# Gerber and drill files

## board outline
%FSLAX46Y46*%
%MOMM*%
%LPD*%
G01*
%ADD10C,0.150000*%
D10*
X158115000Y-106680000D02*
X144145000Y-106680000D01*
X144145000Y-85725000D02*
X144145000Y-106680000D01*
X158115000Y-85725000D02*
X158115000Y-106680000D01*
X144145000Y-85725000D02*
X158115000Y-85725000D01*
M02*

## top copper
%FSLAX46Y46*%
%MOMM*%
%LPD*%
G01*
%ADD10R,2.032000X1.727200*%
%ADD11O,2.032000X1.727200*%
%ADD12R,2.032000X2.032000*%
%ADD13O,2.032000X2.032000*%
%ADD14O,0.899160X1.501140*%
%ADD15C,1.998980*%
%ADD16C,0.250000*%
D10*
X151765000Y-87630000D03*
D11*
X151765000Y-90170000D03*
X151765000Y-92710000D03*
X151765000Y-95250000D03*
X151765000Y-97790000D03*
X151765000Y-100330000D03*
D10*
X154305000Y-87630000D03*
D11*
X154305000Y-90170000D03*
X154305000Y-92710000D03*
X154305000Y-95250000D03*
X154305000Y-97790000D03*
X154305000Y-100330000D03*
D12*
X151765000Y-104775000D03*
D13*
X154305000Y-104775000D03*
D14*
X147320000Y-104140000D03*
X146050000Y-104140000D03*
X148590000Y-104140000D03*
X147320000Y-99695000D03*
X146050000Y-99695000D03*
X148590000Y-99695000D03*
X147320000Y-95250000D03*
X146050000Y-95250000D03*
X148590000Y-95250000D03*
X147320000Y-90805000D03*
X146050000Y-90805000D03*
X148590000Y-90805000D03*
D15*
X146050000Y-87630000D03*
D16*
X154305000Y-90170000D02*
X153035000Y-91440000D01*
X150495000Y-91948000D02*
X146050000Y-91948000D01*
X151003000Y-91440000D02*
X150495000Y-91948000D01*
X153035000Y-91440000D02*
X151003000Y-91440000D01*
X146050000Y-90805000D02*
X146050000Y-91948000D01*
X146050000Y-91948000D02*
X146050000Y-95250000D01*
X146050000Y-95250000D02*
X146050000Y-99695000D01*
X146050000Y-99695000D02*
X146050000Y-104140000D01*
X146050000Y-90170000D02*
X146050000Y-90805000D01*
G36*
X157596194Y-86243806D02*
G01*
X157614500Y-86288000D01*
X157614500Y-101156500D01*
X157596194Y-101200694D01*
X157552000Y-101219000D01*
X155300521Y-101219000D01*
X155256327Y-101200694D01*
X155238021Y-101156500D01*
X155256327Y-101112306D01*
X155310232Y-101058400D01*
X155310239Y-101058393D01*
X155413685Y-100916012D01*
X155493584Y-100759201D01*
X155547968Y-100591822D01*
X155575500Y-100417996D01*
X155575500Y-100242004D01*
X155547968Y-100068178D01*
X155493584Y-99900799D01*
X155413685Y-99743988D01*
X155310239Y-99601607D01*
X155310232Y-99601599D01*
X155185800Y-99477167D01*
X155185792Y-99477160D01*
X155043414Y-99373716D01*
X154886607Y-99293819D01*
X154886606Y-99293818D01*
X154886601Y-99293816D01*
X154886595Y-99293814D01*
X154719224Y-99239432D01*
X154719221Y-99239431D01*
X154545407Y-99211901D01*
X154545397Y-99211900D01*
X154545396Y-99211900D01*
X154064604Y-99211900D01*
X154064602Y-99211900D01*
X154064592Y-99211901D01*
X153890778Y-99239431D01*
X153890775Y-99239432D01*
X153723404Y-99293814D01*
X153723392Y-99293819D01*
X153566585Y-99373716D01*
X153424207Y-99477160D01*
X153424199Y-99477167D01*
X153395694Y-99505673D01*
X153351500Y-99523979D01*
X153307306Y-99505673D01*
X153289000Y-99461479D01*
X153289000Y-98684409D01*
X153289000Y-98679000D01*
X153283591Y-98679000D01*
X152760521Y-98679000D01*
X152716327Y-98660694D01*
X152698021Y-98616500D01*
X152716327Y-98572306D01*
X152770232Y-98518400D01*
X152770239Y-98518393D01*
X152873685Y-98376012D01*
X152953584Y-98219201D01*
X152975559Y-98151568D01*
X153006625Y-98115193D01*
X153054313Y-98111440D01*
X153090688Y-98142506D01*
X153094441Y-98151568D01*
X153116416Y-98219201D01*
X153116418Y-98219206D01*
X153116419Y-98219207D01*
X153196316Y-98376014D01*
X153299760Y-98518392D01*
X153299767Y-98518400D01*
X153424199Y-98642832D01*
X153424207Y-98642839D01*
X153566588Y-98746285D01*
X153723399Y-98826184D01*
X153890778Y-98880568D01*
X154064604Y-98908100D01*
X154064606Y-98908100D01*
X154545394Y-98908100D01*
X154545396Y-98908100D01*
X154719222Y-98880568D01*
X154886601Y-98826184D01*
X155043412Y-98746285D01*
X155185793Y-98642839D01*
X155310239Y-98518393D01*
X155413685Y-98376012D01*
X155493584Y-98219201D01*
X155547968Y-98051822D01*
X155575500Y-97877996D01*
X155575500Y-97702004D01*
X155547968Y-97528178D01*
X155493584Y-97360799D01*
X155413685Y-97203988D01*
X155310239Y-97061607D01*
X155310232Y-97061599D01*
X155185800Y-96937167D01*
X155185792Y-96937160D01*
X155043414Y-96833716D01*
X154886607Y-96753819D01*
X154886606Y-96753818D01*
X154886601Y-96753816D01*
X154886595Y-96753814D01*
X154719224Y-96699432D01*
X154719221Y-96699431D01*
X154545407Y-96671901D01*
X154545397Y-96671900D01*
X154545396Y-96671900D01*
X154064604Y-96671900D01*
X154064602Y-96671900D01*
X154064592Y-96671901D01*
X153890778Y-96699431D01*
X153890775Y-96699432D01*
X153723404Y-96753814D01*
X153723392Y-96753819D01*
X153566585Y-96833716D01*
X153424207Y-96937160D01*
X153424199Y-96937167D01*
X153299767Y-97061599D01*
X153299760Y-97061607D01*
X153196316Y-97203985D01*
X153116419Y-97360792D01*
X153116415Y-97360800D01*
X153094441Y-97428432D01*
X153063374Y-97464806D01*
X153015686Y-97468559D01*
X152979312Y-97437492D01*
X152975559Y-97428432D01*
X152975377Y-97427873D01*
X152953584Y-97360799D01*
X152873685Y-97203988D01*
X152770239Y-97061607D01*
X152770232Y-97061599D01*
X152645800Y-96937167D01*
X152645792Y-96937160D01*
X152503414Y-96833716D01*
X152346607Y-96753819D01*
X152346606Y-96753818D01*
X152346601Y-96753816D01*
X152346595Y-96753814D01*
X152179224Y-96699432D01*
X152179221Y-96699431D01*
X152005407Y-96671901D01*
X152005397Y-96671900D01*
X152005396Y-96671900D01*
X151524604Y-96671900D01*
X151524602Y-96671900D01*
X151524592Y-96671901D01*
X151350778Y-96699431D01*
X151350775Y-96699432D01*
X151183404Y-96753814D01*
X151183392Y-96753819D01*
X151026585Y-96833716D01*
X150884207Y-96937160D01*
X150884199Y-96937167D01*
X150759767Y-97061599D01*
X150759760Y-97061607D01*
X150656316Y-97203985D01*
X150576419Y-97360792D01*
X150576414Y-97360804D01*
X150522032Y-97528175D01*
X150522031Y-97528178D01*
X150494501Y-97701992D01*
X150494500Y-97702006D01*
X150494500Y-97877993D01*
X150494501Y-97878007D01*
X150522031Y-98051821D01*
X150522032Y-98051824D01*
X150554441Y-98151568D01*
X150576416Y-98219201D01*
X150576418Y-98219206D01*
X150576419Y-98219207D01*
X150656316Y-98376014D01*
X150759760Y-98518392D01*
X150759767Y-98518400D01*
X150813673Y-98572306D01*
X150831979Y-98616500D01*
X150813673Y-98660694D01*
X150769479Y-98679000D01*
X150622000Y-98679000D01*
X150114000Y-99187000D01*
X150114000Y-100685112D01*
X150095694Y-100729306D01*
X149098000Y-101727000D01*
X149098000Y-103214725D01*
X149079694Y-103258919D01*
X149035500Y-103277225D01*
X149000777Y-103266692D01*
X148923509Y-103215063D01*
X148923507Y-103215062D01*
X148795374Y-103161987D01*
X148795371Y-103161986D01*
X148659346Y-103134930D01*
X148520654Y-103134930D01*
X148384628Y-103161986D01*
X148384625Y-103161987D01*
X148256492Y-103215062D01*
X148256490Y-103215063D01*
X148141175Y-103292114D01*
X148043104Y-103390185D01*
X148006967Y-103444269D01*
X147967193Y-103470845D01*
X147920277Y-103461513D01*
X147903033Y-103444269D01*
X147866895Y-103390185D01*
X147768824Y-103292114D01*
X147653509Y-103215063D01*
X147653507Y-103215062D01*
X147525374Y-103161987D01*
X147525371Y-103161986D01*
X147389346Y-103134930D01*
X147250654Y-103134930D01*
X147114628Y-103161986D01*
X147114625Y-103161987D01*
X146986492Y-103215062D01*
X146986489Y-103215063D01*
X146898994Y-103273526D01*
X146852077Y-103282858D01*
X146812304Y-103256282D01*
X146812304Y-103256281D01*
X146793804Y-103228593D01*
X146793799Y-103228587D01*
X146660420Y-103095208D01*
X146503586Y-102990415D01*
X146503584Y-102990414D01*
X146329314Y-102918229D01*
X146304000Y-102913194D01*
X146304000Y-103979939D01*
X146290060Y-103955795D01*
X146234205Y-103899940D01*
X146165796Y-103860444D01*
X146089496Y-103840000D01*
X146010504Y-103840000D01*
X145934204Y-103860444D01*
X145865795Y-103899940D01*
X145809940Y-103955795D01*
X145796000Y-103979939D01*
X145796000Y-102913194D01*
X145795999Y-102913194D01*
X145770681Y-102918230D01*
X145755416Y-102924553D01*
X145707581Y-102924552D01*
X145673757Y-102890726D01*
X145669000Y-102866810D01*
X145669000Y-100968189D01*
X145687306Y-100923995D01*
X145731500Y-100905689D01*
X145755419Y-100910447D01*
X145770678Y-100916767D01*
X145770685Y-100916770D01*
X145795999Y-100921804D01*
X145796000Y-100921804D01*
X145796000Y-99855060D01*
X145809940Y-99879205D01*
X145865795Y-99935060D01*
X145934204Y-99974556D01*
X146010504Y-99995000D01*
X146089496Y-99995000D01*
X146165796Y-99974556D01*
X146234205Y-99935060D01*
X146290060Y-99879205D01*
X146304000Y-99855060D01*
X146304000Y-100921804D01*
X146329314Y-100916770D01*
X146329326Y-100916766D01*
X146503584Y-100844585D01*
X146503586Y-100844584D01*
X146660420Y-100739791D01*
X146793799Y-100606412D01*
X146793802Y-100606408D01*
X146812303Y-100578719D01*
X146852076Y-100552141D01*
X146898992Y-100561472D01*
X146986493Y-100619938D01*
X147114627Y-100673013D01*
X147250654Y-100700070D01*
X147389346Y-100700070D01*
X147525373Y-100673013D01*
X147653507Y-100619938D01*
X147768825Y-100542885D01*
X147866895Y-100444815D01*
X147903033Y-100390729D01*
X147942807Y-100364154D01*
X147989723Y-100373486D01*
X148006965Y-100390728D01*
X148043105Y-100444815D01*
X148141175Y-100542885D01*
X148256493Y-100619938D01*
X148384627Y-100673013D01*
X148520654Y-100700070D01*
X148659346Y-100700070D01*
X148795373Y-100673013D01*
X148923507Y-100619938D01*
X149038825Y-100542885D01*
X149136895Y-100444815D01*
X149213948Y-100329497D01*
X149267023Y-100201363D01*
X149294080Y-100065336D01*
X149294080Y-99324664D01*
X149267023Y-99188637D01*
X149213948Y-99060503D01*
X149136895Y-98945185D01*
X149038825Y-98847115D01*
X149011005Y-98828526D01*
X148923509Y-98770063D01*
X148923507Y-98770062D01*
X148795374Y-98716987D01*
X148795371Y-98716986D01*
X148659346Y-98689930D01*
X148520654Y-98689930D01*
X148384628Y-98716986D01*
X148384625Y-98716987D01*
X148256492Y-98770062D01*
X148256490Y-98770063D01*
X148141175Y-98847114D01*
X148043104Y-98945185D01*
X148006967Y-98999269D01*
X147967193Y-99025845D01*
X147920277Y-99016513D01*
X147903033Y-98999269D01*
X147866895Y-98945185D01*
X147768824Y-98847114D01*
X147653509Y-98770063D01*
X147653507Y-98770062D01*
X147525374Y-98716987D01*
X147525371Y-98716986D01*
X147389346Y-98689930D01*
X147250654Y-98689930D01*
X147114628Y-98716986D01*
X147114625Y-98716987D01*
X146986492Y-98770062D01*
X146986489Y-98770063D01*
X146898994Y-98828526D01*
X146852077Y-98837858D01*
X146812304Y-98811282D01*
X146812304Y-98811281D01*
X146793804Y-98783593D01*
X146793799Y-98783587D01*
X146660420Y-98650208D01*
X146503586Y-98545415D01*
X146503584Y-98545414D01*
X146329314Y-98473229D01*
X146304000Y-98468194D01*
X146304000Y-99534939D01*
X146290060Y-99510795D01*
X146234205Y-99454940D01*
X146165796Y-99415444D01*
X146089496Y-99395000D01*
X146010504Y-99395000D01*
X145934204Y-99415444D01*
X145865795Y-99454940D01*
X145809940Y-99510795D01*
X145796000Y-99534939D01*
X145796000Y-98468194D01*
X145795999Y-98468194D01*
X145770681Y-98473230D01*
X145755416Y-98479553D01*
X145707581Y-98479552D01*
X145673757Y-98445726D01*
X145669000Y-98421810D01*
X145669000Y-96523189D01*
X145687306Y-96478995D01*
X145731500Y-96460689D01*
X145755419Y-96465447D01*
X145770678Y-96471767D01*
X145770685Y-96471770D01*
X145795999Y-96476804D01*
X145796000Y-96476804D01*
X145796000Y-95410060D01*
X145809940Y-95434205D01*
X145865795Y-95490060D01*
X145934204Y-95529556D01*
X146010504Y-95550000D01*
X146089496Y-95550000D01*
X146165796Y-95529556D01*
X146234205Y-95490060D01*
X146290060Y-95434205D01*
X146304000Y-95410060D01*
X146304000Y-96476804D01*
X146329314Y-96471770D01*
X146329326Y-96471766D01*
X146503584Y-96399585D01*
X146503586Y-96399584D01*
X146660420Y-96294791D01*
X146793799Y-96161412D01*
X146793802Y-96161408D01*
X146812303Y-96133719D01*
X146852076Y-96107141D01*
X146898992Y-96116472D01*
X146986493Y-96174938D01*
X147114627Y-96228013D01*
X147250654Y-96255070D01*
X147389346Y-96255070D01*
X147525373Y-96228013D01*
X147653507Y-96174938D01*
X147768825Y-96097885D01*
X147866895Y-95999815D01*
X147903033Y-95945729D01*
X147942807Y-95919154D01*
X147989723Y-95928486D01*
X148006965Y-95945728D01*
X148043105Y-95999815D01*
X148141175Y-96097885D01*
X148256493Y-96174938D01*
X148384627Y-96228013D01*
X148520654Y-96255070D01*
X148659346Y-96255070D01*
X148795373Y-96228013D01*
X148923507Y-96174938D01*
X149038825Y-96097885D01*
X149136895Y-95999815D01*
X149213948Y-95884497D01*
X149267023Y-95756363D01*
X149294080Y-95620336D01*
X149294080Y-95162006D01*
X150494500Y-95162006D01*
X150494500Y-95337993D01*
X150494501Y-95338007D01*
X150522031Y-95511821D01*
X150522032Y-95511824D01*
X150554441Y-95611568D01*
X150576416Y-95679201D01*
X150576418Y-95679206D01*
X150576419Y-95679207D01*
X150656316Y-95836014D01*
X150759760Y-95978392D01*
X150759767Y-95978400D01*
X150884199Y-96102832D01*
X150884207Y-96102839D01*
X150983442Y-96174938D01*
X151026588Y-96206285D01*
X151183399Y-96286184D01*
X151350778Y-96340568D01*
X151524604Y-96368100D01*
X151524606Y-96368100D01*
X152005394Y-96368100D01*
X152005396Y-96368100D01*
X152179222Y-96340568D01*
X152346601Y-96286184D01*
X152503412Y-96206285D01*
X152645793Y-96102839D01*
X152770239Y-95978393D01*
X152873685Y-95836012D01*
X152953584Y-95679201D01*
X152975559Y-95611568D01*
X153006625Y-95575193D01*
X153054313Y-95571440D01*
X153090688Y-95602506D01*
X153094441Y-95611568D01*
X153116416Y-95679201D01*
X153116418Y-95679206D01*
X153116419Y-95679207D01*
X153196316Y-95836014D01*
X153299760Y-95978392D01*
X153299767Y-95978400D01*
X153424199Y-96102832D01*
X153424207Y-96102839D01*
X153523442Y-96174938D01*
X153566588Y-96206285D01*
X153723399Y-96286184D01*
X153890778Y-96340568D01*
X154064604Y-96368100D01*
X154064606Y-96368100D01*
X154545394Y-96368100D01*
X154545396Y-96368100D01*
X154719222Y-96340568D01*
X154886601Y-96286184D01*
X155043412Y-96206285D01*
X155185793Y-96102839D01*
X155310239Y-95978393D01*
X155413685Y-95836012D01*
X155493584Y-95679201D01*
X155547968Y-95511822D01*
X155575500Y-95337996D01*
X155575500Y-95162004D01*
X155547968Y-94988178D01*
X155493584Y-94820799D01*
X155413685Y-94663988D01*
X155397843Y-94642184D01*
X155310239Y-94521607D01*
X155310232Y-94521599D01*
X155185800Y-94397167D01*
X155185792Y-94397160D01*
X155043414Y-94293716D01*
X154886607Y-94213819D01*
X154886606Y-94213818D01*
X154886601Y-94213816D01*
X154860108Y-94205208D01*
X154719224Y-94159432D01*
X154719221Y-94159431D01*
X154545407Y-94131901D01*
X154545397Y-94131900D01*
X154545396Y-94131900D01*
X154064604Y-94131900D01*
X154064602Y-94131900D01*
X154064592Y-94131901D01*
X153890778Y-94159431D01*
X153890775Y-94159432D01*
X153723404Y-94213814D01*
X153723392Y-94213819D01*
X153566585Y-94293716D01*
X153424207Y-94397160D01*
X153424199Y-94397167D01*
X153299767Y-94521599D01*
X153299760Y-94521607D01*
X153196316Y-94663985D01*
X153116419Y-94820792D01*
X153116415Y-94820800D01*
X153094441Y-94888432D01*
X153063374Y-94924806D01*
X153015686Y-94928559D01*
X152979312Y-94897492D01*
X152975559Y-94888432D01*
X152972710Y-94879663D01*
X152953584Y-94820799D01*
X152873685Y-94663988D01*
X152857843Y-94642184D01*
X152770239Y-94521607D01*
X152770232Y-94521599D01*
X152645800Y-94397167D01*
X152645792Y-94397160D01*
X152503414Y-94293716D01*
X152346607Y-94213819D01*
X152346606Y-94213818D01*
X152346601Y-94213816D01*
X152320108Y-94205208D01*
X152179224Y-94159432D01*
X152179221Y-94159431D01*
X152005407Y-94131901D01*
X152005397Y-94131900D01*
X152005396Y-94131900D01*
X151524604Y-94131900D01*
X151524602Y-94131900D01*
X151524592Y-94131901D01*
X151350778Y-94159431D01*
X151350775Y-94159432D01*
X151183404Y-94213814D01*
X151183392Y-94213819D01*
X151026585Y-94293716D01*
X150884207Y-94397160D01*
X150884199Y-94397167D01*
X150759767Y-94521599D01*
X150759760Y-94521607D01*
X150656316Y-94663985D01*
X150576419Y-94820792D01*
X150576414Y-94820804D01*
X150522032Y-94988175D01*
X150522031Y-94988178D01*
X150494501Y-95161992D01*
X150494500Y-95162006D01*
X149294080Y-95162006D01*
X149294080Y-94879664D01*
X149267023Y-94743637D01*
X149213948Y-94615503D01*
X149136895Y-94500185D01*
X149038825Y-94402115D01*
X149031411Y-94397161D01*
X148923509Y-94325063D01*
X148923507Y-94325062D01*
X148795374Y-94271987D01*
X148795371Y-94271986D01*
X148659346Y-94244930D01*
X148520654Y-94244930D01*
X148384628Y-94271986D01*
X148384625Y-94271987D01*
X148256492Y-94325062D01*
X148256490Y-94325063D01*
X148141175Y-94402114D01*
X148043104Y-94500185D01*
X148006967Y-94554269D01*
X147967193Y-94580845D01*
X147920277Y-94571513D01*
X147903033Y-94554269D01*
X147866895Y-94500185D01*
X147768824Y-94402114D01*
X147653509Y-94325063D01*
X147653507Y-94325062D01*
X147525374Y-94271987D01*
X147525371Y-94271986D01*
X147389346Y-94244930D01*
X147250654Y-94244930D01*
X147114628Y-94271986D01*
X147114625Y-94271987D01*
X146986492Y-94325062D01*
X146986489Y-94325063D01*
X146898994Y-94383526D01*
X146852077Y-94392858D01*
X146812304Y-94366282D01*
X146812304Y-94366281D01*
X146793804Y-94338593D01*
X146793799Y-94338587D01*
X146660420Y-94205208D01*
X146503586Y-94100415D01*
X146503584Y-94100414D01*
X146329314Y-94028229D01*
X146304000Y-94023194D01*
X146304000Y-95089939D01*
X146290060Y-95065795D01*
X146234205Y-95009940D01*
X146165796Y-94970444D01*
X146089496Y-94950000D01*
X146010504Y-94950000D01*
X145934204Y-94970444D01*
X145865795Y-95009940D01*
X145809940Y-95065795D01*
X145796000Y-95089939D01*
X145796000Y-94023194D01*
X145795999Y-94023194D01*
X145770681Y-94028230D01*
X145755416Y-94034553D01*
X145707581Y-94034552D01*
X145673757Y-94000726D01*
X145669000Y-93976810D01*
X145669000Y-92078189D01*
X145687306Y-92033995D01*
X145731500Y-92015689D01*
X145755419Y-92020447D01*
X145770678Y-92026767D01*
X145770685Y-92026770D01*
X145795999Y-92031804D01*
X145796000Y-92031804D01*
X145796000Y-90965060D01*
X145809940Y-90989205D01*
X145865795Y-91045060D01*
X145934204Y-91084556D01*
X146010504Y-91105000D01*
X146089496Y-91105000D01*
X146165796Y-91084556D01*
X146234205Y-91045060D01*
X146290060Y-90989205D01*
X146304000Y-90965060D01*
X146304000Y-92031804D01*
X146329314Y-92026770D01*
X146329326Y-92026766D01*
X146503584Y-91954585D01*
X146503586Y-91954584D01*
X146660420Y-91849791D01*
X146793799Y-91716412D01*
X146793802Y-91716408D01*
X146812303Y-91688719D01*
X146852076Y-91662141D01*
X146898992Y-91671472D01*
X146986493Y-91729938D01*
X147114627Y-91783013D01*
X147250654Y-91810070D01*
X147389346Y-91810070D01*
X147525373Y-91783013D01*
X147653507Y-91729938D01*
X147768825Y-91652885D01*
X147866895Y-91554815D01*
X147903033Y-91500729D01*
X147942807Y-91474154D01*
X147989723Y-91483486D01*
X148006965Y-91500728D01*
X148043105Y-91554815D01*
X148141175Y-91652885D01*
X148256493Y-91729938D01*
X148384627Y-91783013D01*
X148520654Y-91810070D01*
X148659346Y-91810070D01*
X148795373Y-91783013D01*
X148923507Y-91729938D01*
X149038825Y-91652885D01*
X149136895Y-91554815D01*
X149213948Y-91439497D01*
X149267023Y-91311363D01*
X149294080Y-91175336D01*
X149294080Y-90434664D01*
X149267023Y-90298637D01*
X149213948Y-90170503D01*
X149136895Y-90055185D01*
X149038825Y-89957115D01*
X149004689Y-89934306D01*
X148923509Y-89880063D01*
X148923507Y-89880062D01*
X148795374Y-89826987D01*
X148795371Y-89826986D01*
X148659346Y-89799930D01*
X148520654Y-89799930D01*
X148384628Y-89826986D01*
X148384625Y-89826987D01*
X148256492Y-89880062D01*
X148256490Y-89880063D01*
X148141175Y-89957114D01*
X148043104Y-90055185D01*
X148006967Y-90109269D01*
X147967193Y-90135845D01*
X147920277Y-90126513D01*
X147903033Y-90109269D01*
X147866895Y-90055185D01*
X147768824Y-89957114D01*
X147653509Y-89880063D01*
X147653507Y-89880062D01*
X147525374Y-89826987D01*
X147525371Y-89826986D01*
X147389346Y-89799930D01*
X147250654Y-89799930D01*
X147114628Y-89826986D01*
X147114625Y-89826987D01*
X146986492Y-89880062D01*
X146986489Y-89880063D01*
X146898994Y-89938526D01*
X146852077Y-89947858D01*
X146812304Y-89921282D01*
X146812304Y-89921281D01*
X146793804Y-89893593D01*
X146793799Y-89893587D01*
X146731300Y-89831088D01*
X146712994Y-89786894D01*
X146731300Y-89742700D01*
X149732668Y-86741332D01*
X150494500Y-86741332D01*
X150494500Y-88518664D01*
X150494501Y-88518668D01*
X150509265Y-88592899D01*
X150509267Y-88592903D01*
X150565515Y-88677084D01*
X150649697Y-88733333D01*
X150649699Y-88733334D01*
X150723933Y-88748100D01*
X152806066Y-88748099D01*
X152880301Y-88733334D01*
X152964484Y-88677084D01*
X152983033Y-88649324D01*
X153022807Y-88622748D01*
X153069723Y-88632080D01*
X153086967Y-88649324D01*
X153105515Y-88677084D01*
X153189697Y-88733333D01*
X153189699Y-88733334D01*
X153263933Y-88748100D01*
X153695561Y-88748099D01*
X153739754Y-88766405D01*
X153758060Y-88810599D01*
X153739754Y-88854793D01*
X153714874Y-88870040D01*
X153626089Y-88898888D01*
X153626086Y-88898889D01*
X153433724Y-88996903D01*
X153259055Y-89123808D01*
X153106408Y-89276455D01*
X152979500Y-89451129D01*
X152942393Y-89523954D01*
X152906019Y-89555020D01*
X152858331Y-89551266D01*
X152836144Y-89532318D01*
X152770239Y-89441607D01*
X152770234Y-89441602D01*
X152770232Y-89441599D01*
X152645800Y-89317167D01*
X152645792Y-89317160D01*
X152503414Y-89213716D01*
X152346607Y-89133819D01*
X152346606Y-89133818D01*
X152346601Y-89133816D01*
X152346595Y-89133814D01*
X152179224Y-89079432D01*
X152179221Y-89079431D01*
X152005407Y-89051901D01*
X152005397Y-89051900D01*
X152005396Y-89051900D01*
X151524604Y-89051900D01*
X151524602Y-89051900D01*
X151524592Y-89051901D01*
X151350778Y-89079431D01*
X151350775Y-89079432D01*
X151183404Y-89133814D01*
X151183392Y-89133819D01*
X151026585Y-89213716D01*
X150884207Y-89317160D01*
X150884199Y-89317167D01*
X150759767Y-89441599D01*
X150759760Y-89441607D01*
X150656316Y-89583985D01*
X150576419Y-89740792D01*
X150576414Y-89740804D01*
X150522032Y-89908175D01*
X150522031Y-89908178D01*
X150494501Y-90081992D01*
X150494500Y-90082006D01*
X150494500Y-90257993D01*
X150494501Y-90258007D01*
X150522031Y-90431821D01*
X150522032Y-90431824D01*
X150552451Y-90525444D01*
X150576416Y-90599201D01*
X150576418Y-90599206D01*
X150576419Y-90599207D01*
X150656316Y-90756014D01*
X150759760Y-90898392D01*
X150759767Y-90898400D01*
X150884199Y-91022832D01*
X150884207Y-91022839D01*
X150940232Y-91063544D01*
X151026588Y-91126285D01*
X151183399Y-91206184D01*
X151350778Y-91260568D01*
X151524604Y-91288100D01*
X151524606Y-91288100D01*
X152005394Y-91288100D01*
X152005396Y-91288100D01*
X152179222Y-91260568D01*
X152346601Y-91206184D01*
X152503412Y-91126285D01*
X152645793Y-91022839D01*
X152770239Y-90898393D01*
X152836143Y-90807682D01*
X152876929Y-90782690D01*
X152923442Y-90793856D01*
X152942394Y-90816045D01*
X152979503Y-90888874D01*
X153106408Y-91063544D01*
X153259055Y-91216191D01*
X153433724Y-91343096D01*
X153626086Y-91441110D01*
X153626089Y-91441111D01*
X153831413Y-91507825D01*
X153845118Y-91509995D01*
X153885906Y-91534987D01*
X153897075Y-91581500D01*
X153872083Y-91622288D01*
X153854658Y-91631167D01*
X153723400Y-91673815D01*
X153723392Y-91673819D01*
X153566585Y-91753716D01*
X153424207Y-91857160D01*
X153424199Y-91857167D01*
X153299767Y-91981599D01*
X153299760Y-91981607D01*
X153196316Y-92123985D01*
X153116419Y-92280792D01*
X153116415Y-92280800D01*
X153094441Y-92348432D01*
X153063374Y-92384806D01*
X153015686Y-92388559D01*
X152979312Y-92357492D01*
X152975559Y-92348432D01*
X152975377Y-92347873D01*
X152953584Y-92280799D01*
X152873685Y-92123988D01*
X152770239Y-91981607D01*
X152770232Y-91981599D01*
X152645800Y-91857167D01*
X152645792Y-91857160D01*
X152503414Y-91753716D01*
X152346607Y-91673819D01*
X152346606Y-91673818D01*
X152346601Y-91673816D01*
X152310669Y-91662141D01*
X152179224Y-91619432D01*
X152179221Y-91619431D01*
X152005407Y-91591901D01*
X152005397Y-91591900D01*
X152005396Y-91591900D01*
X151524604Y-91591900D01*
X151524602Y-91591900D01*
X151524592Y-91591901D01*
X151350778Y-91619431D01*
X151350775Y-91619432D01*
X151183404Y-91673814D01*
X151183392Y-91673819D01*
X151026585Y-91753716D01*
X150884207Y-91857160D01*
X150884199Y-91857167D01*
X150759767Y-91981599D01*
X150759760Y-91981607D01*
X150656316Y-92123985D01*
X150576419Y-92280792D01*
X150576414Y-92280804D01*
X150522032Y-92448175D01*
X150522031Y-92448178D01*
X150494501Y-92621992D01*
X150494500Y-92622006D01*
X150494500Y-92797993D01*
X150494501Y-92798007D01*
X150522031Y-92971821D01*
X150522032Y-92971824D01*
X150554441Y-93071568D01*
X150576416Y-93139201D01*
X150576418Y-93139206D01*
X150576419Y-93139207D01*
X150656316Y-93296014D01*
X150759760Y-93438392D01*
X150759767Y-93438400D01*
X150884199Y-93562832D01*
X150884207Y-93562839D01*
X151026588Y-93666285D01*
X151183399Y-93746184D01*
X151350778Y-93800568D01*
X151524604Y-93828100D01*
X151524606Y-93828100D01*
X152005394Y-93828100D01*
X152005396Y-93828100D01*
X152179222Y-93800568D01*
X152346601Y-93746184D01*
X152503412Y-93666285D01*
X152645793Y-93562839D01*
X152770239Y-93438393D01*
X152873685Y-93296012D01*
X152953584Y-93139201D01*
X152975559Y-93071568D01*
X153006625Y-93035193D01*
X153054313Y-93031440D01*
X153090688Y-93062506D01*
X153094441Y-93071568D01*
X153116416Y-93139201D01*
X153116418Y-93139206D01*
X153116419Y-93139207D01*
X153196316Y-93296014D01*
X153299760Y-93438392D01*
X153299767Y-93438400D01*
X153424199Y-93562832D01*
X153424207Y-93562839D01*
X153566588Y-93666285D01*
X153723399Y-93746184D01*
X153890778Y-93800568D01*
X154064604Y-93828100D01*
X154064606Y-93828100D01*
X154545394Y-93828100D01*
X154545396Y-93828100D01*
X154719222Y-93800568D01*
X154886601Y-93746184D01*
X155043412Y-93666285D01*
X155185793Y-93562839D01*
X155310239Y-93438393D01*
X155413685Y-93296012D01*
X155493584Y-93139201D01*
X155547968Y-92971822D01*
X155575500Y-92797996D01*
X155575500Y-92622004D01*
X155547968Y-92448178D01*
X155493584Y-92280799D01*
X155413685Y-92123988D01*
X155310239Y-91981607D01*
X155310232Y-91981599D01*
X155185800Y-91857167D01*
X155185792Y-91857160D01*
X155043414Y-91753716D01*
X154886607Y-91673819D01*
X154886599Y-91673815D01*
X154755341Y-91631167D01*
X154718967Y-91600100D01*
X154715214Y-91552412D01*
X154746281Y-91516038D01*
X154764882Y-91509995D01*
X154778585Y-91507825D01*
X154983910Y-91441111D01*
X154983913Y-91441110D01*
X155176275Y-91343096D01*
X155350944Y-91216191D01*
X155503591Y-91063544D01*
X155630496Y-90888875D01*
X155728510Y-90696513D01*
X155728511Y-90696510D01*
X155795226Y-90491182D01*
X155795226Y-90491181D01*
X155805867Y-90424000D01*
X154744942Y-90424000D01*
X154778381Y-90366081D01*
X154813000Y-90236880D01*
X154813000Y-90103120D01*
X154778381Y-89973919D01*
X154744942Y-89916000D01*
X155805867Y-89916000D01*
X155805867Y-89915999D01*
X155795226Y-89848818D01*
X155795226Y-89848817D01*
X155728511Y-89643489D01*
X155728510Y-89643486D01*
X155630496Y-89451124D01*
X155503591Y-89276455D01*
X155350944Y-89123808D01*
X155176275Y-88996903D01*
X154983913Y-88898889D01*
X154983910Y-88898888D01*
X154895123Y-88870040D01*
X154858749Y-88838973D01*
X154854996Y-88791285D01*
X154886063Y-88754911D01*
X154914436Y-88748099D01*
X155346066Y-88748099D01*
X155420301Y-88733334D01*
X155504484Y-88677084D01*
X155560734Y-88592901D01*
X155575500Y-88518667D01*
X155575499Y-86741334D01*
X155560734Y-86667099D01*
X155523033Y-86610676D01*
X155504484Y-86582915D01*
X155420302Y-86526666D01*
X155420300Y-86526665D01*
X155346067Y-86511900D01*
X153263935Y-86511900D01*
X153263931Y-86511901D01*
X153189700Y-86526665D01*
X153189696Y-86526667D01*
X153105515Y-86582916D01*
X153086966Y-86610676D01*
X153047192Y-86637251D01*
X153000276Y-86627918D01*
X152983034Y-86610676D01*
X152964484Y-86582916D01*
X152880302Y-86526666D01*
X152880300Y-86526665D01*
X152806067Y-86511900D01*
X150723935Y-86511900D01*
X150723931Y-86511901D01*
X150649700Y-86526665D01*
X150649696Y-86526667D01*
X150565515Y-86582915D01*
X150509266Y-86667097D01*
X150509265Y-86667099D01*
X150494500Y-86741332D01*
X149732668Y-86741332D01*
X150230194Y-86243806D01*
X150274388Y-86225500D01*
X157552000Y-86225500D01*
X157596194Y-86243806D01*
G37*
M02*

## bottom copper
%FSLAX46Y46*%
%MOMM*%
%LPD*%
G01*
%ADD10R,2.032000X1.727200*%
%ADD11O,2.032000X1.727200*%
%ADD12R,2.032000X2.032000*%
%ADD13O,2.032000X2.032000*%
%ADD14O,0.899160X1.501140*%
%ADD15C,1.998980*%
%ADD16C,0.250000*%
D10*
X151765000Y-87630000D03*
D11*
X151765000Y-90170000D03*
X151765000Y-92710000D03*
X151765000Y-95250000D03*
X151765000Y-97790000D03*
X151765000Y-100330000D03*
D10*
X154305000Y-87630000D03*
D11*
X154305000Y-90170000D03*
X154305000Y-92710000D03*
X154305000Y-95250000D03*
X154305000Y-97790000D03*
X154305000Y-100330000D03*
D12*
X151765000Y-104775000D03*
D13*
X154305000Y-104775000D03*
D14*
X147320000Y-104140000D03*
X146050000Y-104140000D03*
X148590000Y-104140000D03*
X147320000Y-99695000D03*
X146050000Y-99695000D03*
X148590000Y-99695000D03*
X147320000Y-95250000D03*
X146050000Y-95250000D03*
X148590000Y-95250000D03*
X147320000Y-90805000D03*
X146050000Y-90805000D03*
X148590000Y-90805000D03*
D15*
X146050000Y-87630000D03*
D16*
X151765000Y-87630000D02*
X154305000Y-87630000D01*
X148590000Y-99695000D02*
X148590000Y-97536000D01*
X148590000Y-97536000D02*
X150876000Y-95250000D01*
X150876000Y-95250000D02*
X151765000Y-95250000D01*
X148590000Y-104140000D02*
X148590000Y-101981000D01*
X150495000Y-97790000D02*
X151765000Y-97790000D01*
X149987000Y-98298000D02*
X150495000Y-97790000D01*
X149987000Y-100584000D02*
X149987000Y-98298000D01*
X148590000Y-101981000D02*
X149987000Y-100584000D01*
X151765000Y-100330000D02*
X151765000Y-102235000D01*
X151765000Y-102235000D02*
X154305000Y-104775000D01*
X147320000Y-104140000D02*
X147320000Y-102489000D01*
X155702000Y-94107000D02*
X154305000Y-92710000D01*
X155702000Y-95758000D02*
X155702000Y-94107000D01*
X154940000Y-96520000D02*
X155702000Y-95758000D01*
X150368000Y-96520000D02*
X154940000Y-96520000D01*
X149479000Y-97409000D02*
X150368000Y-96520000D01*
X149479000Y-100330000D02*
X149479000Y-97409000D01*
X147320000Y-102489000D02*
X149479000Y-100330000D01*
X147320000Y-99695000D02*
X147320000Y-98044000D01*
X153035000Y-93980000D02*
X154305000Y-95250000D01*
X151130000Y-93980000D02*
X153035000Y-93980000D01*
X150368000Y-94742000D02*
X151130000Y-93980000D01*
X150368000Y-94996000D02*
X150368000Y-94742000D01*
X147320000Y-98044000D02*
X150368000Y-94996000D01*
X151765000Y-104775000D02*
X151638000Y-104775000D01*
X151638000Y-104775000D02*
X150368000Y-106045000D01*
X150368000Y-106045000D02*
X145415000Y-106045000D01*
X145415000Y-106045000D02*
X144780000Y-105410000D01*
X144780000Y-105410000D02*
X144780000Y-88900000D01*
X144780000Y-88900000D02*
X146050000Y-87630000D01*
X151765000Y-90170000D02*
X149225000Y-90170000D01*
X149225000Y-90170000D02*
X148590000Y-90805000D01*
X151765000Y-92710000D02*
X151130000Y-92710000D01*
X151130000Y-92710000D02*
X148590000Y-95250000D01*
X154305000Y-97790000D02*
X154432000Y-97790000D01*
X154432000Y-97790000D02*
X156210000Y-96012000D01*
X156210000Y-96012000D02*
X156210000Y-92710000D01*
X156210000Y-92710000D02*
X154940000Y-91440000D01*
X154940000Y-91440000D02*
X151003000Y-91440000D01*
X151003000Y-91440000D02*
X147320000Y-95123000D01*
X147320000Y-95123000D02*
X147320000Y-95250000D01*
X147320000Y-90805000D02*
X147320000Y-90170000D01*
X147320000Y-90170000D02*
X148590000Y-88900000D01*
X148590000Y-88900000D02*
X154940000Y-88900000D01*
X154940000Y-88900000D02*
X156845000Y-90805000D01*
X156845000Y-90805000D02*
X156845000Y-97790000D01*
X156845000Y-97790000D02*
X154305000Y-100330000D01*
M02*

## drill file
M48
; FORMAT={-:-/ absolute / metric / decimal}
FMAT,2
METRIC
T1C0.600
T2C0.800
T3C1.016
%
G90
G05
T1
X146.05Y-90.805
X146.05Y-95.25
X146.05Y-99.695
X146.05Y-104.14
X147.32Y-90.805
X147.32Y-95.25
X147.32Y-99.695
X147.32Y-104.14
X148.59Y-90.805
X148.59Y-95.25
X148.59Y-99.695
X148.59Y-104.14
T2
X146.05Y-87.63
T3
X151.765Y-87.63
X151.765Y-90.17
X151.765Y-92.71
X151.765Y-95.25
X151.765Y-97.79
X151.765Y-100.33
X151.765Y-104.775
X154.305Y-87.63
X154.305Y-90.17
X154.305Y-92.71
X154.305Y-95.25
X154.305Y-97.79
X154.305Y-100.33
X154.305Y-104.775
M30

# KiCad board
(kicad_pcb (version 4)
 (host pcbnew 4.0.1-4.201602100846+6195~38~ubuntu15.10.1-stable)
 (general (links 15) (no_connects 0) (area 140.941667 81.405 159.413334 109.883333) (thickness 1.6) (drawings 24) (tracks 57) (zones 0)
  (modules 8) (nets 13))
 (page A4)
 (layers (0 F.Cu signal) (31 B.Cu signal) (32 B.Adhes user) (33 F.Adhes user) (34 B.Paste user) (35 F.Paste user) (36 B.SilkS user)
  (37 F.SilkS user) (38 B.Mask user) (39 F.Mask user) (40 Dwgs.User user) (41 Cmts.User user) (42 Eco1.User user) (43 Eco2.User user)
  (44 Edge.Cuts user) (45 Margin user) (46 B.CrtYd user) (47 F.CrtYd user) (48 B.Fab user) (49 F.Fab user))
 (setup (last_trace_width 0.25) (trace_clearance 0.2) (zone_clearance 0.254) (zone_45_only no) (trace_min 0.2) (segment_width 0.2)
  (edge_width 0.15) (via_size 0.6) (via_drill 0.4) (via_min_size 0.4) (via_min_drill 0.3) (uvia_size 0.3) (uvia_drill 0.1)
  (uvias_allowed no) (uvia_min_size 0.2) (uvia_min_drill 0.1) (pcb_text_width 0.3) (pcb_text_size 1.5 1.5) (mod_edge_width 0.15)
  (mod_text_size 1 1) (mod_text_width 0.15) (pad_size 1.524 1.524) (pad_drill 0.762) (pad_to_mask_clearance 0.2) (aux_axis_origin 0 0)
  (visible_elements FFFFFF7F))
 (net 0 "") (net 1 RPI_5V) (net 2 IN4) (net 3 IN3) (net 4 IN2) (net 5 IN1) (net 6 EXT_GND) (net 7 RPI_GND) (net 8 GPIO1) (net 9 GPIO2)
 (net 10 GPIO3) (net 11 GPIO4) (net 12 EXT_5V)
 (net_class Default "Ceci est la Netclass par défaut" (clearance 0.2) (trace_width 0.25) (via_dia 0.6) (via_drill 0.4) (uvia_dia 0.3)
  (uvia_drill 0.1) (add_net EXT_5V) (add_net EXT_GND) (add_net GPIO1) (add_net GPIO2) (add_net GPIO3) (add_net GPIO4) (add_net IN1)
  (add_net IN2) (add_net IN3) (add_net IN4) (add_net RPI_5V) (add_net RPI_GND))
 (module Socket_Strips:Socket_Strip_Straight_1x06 (layer B.Cu) (at 151.765 87.63 270)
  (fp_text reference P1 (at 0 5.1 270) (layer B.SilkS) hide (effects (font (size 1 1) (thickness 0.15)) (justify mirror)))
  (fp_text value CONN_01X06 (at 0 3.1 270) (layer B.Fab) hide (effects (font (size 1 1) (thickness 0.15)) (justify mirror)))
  (pad 1 thru_hole rect (at 0 0 270) (size 1.7272 2.032) (drill 1.016) (layers *.Cu *.Mask B.SilkS) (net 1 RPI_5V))
  (pad 2 thru_hole oval (at 2.54 0 270) (size 1.7272 2.032) (drill 1.016) (layers *.Cu *.Mask B.SilkS) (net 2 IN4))
  (pad 3 thru_hole oval (at 5.08 0 270) (size 1.7272 2.032) (drill 1.016) (layers *.Cu *.Mask B.SilkS) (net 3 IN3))
  (pad 4 thru_hole oval (at 7.62 0 270) (size 1.7272 2.032) (drill 1.016) (layers *.Cu *.Mask B.SilkS) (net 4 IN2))
  (pad 5 thru_hole oval (at 10.16 0 270) (size 1.7272 2.032) (drill 1.016) (layers *.Cu *.Mask B.SilkS) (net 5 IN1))
  (pad 6 thru_hole oval (at 12.7 0 270) (size 1.7272 2.032) (drill 1.016) (layers *.Cu *.Mask B.SilkS) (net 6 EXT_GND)))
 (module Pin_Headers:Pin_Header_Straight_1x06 (layer F.Cu) (at 154.305 87.63)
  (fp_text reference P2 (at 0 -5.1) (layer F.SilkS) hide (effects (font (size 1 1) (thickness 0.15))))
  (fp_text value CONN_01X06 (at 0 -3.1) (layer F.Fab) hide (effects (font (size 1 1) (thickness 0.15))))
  (pad 1 thru_hole rect (at 0 0) (size 2.032 1.7272) (drill 1.016) (layers *.Cu *.Mask F.SilkS) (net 1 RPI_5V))
  (pad 2 thru_hole oval (at 0 2.54) (size 2.032 1.7272) (drill 1.016) (layers *.Cu *.Mask F.SilkS) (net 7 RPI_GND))
  (pad 3 thru_hole oval (at 0 5.08) (size 2.032 1.7272) (drill 1.016) (layers *.Cu *.Mask F.SilkS) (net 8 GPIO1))
  (pad 4 thru_hole oval (at 0 7.62) (size 2.032 1.7272) (drill 1.016) (layers *.Cu *.Mask F.SilkS) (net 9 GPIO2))
  (pad 5 thru_hole oval (at 0 10.16) (size 2.032 1.7272) (drill 1.016) (layers *.Cu *.Mask F.SilkS) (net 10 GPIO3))
  (pad 6 thru_hole oval (at 0 12.7) (size 2.032 1.7272) (drill 1.016) (layers *.Cu *.Mask F.SilkS) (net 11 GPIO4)))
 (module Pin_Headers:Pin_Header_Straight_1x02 (layer F.Cu) (at 151.765 104.775 90)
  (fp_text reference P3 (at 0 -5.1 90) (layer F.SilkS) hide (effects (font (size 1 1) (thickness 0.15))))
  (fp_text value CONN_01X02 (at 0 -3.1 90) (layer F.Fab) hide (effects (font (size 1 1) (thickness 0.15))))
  (pad 1 thru_hole rect (at 0 0 90) (size 2.032 2.032) (drill 1.016) (layers *.Cu *.Mask F.SilkS) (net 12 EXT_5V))
  (pad 2 thru_hole oval (at 0 2.54 90) (size 2.032 2.032) (drill 1.016) (layers *.Cu *.Mask F.SilkS) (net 6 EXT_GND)))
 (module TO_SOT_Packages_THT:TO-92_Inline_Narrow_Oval (layer F.Cu) (at 148.59 104.14 180)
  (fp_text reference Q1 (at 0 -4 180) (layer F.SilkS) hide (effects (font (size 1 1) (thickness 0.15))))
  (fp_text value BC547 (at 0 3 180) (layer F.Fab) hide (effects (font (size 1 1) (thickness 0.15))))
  (pad 2 thru_hole oval (at 1.27 0) (size 0.89916 1.50114) (drill 0.6) (layers *.Cu *.Mask F.SilkS) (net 8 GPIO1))
  (pad 3 thru_hole oval (at 2.54 0) (size 0.89916 1.50114) (drill 0.6) (layers *.Cu *.Mask F.SilkS) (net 7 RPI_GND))
  (pad 1 thru_hole oval (at 0 0) (size 0.89916 1.50114) (drill 0.6) (layers *.Cu *.Mask F.SilkS) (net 5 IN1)))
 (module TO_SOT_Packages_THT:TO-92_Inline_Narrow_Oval (layer F.Cu) (at 148.59 99.695 180)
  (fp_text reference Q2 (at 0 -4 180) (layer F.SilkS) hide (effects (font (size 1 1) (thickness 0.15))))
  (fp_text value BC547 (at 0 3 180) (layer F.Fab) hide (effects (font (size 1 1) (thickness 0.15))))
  (pad 2 thru_hole oval (at 1.27 0) (size 0.89916 1.50114) (drill 0.6) (layers *.Cu *.Mask F.SilkS) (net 9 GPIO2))
  (pad 3 thru_hole oval (at 2.54 0) (size 0.89916 1.50114) (drill 0.6) (layers *.Cu *.Mask F.SilkS) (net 7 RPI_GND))
  (pad 1 thru_hole oval (at 0 0) (size 0.89916 1.50114) (drill 0.6) (layers *.Cu *.Mask F.SilkS) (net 4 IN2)))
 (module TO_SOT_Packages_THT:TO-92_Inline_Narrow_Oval (layer F.Cu) (at 148.59 95.25 180)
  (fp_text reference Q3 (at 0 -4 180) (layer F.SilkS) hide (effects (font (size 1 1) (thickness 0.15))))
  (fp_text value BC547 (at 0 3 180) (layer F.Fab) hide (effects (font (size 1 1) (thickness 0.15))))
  (pad 2 thru_hole oval (at 1.27 0) (size 0.89916 1.50114) (drill 0.6) (layers *.Cu *.Mask F.SilkS) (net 10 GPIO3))
  (pad 3 thru_hole oval (at 2.54 0) (size 0.89916 1.50114) (drill 0.6) (layers *.Cu *.Mask F.SilkS) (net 7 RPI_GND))
  (pad 1 thru_hole oval (at 0 0) (size 0.89916 1.50114) (drill 0.6) (layers *.Cu *.Mask F.SilkS) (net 3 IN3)))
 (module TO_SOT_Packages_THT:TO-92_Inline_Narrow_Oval (layer F.Cu) (at 148.59 90.805 180)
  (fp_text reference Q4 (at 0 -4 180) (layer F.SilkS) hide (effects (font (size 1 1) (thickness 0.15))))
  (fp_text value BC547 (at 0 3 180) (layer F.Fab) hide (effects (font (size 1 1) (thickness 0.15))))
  (pad 2 thru_hole oval (at 1.27 0) (size 0.89916 1.50114) (drill 0.6) (layers *.Cu *.Mask F.SilkS) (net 11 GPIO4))
  (pad 3 thru_hole oval (at 2.54 0) (size 0.89916 1.50114) (drill 0.6) (layers *.Cu *.Mask F.SilkS) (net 7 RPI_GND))
  (pad 1 thru_hole oval (at 0 0) (size 0.89916 1.50114) (drill 0.6) (layers *.Cu *.Mask F.SilkS) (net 2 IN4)))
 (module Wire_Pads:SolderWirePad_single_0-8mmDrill (layer F.Cu) (at 146.05 87.63)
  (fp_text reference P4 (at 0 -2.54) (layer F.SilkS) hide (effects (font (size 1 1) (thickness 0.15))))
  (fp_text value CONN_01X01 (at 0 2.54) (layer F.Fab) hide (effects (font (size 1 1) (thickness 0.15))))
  (pad 1 thru_hole circle (at 0 0) (size 1.99898 1.99898) (drill 0.8001) (layers *.Cu *.Mask F.SilkS) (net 12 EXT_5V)))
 (gr_line (start 158.115 106.68) (end 144.145 106.68) (angle 90) (layer Edge.Cuts) (width 0.15))
 (gr_line (start 144.145 85.725) (end 144.145 106.68) (angle 90) (layer Edge.Cuts) (width 0.15))
 (gr_line (start 158.115 85.725) (end 158.115 106.68) (angle 90) (layer Edge.Cuts) (width 0.15))
 (gr_line (start 144.145 85.725) (end 158.115 85.725) (angle 90) (layer Edge.Cuts) (width 0.15))
 (segment (start 151.765 87.63) (end 154.305 87.63) (width 0.25) (layer B.Cu) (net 1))
 (segment (start 148.59 99.695) (end 148.59 97.536) (width 0.25) (layer B.Cu) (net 4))
 (segment (start 148.59 97.536) (end 150.876 95.25) (width 0.25) (layer B.Cu) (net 4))
 (segment (start 150.876 95.25) (end 151.765 95.25) (width 0.25) (layer B.Cu) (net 4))
 (segment (start 148.59 104.14) (end 148.59 101.981) (width 0.25) (layer B.Cu) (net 5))
 (segment (start 150.495 97.79) (end 151.765 97.79) (width 0.25) (layer B.Cu) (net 5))
 (segment (start 149.987 98.298) (end 150.495 97.79) (width 0.25) (layer B.Cu) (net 5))
 (segment (start 149.987 100.584) (end 149.987 98.298) (width 0.25) (layer B.Cu) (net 5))
 (segment (start 148.59 101.981) (end 149.987 100.584) (width 0.25) (layer B.Cu) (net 5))
 (segment (start 151.765 100.33) (end 151.765 102.235) (width 0.25) (layer B.Cu) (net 6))
 (segment (start 151.765 102.235) (end 154.305 104.775) (width 0.25) (layer B.Cu) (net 6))
 (segment (start 154.305 90.17) (end 153.035 91.44) (width 0.25) (layer F.Cu) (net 7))
 (segment (start 150.495 91.948) (end 146.05 91.948) (width 0.25) (layer F.Cu) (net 7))
 (segment (start 151.003 91.44) (end 150.495 91.948) (width 0.25) (layer F.Cu) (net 7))
 (segment (start 153.035 91.44) (end 151.003 91.44) (width 0.25) (layer F.Cu) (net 7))
 (segment (start 146.05 90.805) (end 146.05 91.948) (width 0.25) (layer F.Cu) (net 7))
 (segment (start 146.05 91.948) (end 146.05 95.25) (width 0.25) (layer F.Cu) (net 7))
 (segment (start 146.05 95.25) (end 146.05 99.695) (width 0.25) (layer F.Cu) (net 7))
 (segment (start 146.05 99.695) (end 146.05 104.14) (width 0.25) (layer F.Cu) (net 7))
 (segment (start 146.05 90.17) (end 146.05 90.805) (width 0.25) (layer F.Cu) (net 7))
 (segment (start 147.32 104.14) (end 147.32 102.489) (width 0.25) (layer B.Cu) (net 8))
 (segment (start 155.702 94.107) (end 154.305 92.71) (width 0.25) (layer B.Cu) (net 8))
 (segment (start 155.702 95.758) (end 155.702 94.107) (width 0.25) (layer B.Cu) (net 8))
 (segment (start 154.94 96.52) (end 155.702 95.758) (width 0.25) (layer B.Cu) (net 8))
 (segment (start 150.368 96.52) (end 154.94 96.52) (width 0.25) (layer B.Cu) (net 8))
 (segment (start 149.479 97.409) (end 150.368 96.52) (width 0.25) (layer B.Cu) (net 8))
 (segment (start 149.479 100.33) (end 149.479 97.409) (width 0.25) (layer B.Cu) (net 8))
 (segment (start 147.32 102.489) (end 149.479 100.33) (width 0.25) (layer B.Cu) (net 8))
 (segment (start 147.32 99.695) (end 147.32 98.044) (width 0.25) (layer B.Cu) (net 9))
 (segment (start 153.035 93.98) (end 154.305 95.25) (width 0.25) (layer B.Cu) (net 9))
 (segment (start 151.13 93.98) (end 153.035 93.98) (width 0.25) (layer B.Cu) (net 9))
 (segment (start 150.368 94.742) (end 151.13 93.98) (width 0.25) (layer B.Cu) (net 9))
 (segment (start 150.368 94.996) (end 150.368 94.742) (width 0.25) (layer B.Cu) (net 9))
 (segment (start 147.32 98.044) (end 150.368 94.996) (width 0.25) (layer B.Cu) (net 9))
 (segment (start 151.765 104.775) (end 151.638 104.775) (width 0.25) (layer B.Cu) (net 12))
 (segment (start 151.638 104.775) (end 150.368 106.045) (width 0.25) (layer B.Cu) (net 12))
 (segment (start 150.368 106.045) (end 145.415 106.045) (width 0.25) (layer B.Cu) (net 12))
 (segment (start 145.415 106.045) (end 144.78 105.41) (width 0.25) (layer B.Cu) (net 12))
 (segment (start 144.78 105.41) (end 144.78 88.9) (width 0.25) (layer B.Cu) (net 12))
 (segment (start 144.78 88.9) (end 146.05 87.63) (width 0.25) (layer B.Cu) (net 12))
 (segment (start 151.765 90.17) (end 149.225 90.17) (width 0.25) (layer B.Cu) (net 2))
 (segment (start 149.225 90.17) (end 148.59 90.805) (width 0.25) (layer B.Cu) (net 2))
 (segment (start 151.765 92.71) (end 151.13 92.71) (width 0.25) (layer B.Cu) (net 3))
 (segment (start 151.13 92.71) (end 148.59 95.25) (width 0.25) (layer B.Cu) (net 3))
 (segment (start 154.305 97.79) (end 154.432 97.79) (width 0.25) (layer B.Cu) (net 10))
 (segment (start 154.432 97.79) (end 156.21 96.012) (width 0.25) (layer B.Cu) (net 10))
 (segment (start 156.21 96.012) (end 156.21 92.71) (width 0.25) (layer B.Cu) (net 10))
 (segment (start 156.21 92.71) (end 154.94 91.44) (width 0.25) (layer B.Cu) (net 10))
 (segment (start 154.94 91.44) (end 151.003 91.44) (width 0.25) (layer B.Cu) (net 10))
 (segment (start 151.003 91.44) (end 147.32 95.123) (width 0.25) (layer B.Cu) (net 10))
 (segment (start 147.32 95.123) (end 147.32 95.25) (width 0.25) (layer B.Cu) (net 10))
 (segment (start 147.32 90.805) (end 147.32 90.17) (width 0.25) (layer B.Cu) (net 11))
 (segment (start 147.32 90.17) (end 148.59 88.9) (width 0.25) (layer B.Cu) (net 11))
 (segment (start 148.59 88.9) (end 154.94 88.9) (width 0.25) (layer B.Cu) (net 11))
 (segment (start 154.94 88.9) (end 156.845 90.805) (width 0.25) (layer B.Cu) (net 11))
 (segment (start 156.845 90.805) (end 156.845 97.79) (width 0.25) (layer B.Cu) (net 11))
 (segment (start 156.845 97.79) (end 154.305 100.33) (width 0.25) (layer B.Cu) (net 11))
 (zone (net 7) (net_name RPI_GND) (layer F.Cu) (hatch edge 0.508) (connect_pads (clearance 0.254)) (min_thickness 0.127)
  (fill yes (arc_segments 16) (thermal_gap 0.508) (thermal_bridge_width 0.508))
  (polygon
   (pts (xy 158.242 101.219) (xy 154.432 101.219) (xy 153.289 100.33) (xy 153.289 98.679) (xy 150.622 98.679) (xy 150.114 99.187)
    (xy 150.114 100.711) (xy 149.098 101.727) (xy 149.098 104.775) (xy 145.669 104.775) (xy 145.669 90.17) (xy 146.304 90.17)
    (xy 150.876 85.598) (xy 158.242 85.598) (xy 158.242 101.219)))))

